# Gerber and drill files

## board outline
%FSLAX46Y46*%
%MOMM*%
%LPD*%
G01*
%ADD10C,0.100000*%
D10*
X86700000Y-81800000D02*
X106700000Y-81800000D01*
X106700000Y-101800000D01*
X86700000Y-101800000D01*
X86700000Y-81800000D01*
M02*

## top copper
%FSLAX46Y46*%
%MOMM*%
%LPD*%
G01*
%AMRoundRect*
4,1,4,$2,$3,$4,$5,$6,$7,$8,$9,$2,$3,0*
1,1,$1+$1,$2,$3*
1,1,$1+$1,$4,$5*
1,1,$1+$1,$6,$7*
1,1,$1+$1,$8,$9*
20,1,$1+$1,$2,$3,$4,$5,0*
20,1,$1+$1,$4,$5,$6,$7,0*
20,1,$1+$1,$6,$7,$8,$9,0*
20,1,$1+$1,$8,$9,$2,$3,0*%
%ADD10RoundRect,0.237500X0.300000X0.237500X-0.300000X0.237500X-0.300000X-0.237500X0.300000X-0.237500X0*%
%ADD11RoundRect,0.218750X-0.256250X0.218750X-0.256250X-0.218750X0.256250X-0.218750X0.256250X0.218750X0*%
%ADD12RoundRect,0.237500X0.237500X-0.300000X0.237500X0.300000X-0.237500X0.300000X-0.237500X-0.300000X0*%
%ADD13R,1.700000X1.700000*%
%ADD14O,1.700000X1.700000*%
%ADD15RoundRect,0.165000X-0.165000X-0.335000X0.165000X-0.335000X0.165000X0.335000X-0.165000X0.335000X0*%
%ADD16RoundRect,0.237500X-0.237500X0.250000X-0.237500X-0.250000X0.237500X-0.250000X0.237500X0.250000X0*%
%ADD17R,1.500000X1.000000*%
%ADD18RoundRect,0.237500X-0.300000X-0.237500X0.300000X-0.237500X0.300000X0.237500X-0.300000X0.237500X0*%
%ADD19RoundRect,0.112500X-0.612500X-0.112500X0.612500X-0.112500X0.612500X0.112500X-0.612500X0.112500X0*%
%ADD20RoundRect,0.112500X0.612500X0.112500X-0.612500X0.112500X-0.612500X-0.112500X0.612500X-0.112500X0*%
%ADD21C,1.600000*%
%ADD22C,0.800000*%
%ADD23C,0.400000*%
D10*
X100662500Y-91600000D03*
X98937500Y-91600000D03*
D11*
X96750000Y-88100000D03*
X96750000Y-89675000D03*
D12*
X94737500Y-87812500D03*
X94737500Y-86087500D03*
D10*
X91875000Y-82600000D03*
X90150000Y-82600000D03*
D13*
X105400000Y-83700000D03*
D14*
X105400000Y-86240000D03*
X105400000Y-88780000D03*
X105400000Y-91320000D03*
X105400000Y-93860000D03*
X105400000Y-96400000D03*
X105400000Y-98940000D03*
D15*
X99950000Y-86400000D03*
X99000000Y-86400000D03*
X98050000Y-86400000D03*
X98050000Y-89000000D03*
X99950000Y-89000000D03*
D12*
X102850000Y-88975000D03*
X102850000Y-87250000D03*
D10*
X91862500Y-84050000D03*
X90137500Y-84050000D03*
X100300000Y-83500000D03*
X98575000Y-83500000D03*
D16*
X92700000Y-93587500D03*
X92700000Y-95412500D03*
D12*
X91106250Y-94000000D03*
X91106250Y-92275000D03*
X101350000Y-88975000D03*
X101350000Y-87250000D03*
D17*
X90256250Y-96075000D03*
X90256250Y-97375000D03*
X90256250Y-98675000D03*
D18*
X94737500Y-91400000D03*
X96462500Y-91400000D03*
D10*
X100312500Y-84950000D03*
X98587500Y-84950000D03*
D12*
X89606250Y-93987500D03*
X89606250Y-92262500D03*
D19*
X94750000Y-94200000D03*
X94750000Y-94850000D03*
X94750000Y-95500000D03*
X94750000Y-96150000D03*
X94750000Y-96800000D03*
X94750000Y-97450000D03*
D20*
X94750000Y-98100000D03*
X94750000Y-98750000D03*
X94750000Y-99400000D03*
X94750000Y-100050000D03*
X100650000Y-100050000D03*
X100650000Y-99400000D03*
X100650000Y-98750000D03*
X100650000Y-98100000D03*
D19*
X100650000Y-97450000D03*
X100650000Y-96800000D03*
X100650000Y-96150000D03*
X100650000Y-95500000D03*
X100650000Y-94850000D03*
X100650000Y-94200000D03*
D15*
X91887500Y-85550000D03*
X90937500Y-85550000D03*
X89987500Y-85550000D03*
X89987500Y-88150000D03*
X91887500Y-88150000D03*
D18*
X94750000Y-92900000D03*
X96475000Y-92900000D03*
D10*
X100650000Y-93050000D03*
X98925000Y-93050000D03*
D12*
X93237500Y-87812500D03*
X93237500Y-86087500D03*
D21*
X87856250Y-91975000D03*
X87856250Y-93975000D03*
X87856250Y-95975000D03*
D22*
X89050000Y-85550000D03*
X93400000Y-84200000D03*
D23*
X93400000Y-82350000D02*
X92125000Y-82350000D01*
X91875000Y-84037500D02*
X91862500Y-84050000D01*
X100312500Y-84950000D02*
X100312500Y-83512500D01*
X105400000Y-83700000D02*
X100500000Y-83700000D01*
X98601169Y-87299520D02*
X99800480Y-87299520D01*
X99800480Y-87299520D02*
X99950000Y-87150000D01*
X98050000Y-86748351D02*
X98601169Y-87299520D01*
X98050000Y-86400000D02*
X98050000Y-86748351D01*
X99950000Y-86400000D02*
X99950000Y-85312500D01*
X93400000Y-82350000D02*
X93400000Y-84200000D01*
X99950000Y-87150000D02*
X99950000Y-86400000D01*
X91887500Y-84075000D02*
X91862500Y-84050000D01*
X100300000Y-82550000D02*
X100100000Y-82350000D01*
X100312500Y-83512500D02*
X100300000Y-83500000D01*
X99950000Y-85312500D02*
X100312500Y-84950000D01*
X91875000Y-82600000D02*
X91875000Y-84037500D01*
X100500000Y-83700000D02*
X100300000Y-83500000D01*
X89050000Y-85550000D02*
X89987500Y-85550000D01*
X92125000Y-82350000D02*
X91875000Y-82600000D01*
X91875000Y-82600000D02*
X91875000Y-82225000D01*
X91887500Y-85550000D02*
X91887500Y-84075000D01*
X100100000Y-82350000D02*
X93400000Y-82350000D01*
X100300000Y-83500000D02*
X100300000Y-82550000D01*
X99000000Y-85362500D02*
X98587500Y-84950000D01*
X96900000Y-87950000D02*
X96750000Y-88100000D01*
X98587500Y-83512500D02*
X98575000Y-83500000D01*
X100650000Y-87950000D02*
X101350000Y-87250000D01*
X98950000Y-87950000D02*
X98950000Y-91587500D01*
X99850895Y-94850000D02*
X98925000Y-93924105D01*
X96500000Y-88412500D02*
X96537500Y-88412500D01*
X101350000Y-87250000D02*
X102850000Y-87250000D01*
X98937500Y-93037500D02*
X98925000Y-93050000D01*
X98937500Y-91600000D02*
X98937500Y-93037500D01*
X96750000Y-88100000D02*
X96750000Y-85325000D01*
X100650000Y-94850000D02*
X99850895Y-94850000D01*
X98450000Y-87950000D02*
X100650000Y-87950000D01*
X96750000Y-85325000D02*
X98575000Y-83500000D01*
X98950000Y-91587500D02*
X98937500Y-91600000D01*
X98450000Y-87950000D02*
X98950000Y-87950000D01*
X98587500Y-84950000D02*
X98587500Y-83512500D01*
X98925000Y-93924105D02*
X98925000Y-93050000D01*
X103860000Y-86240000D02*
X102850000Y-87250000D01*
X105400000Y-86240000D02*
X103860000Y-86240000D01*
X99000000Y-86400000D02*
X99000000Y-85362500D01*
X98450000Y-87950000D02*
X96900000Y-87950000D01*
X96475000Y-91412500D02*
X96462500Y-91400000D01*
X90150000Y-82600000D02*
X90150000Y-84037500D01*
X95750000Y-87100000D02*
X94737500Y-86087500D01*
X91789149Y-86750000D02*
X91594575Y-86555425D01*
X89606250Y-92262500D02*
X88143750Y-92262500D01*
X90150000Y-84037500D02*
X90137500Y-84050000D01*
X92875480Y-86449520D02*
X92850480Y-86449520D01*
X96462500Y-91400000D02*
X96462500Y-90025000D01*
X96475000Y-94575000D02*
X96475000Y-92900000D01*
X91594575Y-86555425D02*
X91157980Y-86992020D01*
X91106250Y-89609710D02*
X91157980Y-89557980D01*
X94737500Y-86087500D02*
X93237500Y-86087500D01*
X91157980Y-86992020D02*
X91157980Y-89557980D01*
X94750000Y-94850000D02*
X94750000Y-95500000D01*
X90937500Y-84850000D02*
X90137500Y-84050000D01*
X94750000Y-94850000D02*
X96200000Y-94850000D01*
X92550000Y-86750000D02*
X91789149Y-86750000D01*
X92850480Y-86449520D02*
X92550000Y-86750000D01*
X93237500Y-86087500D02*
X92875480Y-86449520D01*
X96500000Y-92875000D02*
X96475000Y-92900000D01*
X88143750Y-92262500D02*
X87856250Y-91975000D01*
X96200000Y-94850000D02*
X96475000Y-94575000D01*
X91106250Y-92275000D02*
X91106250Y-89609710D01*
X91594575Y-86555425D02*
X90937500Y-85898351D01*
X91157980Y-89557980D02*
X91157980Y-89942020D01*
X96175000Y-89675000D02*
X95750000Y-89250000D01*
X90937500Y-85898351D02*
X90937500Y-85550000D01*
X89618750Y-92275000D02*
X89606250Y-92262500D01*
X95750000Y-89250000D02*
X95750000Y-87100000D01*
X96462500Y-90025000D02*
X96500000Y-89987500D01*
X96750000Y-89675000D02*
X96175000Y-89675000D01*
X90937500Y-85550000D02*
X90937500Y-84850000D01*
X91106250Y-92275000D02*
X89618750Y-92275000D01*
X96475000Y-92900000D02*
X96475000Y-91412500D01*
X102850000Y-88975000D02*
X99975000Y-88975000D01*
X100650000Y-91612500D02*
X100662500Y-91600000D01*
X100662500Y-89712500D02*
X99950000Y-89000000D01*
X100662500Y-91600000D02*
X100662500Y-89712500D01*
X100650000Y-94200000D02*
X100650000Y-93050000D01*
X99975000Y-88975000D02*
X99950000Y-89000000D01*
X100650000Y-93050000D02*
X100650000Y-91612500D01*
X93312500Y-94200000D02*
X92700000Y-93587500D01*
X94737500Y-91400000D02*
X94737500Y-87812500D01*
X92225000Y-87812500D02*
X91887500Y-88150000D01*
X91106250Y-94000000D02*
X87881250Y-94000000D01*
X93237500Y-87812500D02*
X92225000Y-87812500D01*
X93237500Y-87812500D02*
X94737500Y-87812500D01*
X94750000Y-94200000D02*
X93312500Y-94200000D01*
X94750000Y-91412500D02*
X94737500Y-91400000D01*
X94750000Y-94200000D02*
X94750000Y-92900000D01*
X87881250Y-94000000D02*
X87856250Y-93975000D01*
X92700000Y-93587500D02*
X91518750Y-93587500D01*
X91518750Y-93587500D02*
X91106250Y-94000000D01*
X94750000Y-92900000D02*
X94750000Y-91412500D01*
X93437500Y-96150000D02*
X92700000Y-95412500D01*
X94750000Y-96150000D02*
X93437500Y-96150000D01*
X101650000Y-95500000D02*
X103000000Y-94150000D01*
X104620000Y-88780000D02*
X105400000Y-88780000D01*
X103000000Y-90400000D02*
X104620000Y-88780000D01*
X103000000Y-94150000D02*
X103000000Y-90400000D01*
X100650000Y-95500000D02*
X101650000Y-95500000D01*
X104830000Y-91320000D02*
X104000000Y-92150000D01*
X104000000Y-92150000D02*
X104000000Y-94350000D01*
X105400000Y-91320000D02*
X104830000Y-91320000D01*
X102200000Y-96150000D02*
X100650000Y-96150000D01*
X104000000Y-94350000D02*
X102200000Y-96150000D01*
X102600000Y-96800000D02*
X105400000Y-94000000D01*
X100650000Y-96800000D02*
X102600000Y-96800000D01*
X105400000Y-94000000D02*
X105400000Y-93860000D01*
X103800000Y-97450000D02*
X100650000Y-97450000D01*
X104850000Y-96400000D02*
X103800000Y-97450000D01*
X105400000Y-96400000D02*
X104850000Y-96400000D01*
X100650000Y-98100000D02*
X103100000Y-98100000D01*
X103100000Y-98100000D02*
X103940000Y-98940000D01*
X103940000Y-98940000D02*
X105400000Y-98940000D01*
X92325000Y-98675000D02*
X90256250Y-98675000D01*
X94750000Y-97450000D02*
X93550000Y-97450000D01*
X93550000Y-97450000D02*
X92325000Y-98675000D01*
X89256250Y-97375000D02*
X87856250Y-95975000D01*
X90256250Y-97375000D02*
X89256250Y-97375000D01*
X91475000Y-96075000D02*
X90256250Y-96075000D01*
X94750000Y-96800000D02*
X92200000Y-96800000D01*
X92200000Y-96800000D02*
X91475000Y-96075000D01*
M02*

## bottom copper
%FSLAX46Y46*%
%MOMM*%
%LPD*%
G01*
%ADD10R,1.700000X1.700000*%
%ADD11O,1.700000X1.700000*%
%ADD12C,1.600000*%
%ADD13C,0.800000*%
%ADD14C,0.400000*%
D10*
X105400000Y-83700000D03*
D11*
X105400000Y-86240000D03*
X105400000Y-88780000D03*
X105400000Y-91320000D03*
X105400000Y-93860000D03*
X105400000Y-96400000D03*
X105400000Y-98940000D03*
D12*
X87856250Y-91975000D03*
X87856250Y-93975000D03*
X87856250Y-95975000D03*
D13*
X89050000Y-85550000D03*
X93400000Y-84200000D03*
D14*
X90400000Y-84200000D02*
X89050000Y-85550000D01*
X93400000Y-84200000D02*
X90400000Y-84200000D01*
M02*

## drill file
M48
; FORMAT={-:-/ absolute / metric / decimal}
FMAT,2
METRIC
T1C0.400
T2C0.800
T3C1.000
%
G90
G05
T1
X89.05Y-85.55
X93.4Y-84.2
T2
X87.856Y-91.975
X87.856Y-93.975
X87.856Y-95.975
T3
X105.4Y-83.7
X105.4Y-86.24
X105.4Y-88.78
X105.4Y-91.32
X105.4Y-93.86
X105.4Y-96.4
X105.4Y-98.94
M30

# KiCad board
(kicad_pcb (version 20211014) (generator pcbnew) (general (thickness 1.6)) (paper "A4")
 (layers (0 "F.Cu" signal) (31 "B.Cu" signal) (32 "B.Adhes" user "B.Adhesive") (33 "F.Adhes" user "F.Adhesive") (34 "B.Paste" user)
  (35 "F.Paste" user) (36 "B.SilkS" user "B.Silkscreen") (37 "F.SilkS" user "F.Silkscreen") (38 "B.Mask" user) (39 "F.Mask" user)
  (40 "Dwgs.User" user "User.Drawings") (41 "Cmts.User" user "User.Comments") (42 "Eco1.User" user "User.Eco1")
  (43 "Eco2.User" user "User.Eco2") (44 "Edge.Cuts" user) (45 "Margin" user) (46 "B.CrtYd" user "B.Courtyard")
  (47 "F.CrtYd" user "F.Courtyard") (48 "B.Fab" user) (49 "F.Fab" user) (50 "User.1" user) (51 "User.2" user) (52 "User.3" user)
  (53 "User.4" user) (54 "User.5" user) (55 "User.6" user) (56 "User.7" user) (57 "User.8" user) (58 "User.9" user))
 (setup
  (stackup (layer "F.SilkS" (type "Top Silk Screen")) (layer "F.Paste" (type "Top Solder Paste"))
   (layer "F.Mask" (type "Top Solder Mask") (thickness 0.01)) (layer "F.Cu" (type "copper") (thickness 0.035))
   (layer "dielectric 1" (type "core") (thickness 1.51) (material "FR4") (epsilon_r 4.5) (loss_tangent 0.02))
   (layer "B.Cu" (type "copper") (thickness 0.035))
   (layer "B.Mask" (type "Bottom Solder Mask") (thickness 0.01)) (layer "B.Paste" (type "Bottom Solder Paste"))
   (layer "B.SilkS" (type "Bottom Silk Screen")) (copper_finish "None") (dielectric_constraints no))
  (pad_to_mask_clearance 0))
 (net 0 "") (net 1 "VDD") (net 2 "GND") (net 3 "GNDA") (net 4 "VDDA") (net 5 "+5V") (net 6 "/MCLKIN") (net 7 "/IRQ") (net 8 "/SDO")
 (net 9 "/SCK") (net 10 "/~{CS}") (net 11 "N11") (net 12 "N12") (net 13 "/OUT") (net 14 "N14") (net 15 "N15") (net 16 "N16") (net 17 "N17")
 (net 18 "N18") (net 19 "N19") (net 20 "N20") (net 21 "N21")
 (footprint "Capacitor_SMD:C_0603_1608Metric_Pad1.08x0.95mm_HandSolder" (layer "F.Cu") (at 99.8 91.6 180)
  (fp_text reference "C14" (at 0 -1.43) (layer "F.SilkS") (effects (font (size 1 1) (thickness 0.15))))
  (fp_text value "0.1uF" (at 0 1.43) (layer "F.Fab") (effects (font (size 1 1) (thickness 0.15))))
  (pad "1" smd roundrect locked (at -0.8625 0 180) (size 1.075 0.95) (layers "F.Cu" "F.Paste" "F.Mask") (roundrect_rratio 0.25)
   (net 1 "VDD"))
  (pad "2" smd roundrect locked (at 0.8625 0 180) (size 1.075 0.95) (layers "F.Cu" "F.Paste" "F.Mask") (roundrect_rratio 0.25) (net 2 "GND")))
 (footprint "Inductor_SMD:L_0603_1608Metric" (layer "F.Cu") (at 96.75 88.8875 -90)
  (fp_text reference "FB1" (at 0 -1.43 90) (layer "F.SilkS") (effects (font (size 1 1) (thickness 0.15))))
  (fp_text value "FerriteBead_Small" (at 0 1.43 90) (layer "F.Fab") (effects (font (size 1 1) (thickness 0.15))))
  (pad "1" smd roundrect locked (at -0.7875 0 270) (size 0.875 0.95) (layers "F.Cu" "F.Paste" "F.Mask") (roundrect_rratio 0.25)
   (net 2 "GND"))
  (pad "2" smd roundrect locked (at 0.7875 0 270) (size 0.875 0.95) (layers "F.Cu" "F.Paste" "F.Mask") (roundrect_rratio 0.25)
   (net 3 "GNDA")))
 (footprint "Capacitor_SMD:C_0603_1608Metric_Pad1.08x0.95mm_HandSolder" (layer "F.Cu") (at 94.7375 86.95 90)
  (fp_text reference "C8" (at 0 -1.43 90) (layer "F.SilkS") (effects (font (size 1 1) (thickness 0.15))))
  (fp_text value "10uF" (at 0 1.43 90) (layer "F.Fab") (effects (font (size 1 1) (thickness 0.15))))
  (pad "1" smd roundrect locked (at -0.8625 0 90) (size 1.075 0.95) (layers "F.Cu" "F.Paste" "F.Mask") (roundrect_rratio 0.25)
   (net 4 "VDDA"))
  (pad "2" smd roundrect locked (at 0.8625 0 90) (size 1.075 0.95) (layers "F.Cu" "F.Paste" "F.Mask") (roundrect_rratio 0.25) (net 3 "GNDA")))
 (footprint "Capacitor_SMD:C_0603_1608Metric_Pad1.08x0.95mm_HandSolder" (layer "F.Cu") (at 91.0125 82.6 180)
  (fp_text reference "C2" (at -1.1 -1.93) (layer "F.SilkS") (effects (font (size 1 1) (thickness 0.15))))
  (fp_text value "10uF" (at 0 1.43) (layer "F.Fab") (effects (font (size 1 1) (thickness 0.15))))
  (pad "1" smd roundrect locked (at -0.8625 0 180) (size 1.075 0.95) (layers "F.Cu" "F.Paste" "F.Mask") (roundrect_rratio 0.25)
   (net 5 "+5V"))
  (pad "2" smd roundrect locked (at 0.8625 0 180) (size 1.075 0.95) (layers "F.Cu" "F.Paste" "F.Mask") (roundrect_rratio 0.25)
   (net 3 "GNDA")))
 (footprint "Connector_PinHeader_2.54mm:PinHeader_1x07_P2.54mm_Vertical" (layer "F.Cu") (at 105.4 83.7)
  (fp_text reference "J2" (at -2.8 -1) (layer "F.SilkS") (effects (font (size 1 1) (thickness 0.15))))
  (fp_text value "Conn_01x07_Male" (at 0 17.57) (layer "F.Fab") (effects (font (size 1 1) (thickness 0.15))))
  (pad "1" thru_hole rect locked (at 0 0) (size 1.7 1.7) (drill 1) (layers *.Cu *.Mask) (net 5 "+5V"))
  (pad "2" thru_hole oval locked (at 0 2.54) (size 1.7 1.7) (drill 1) (layers *.Cu *.Mask) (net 2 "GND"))
  (pad "3" thru_hole oval locked (at 0 5.08) (size 1.7 1.7) (drill 1) (layers *.Cu *.Mask) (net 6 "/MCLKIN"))
  (pad "4" thru_hole oval locked (at 0 7.62) (size 1.7 1.7) (drill 1) (layers *.Cu *.Mask) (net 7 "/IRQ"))
  (pad "5" thru_hole oval locked (at 0 10.16) (size 1.7 1.7) (drill 1) (layers *.Cu *.Mask) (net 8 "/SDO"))
  (pad "6" thru_hole oval locked (at 0 12.7) (size 1.7 1.7) (drill 1) (layers *.Cu *.Mask) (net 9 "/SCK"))
  (pad "7" thru_hole oval locked (at 0 15.24) (size 1.7 1.7) (drill 1) (layers *.Cu *.Mask) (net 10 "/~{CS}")))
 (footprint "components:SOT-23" (layer "F.Cu") (at 99 89)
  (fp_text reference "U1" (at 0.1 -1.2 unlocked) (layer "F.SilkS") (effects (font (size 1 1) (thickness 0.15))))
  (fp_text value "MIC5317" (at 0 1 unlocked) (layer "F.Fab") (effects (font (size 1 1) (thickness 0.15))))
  (pad "1" smd roundrect (at 0.95 -2.6) (size 0.66 1) (layers "F.Cu" "F.Paste" "F.Mask") (roundrect_rratio 0.25) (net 5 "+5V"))
  (pad "2" smd roundrect (at 0 -2.6) (size 0.66 1) (layers "F.Cu" "F.Paste" "F.Mask") (roundrect_rratio 0.25) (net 2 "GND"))
  (pad "3" smd roundrect (at -0.95 -2.6) (size 0.66 1) (layers "F.Cu" "F.Paste" "F.Mask") (roundrect_rratio 0.25) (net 5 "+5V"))
  (pad "4" smd roundrect (at -0.95 0) (size 0.66 1) (layers "F.Cu" "F.Paste" "F.Mask") (roundrect_rratio 0.25))
  (pad "5" smd roundrect (at 0.95 0) (size 0.66 1) (layers "F.Cu" "F.Paste" "F.Mask") (roundrect_rratio 0.25) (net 1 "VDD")))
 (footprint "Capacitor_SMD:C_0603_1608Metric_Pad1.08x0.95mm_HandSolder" (layer "F.Cu") (at 102.85 88.1125 90)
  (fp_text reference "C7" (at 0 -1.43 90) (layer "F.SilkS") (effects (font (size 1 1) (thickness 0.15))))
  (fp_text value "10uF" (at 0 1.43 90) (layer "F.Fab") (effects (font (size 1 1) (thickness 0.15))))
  (pad "1" smd roundrect locked (at -0.8625 0 90) (size 1.075 0.95) (layers "F.Cu" "F.Paste" "F.Mask") (roundrect_rratio 0.25) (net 1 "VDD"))
  (pad "2" smd roundrect locked (at 0.8625 0 90) (size 1.075 0.95) (layers "F.Cu" "F.Paste" "F.Mask") (roundrect_rratio 0.25) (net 2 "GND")))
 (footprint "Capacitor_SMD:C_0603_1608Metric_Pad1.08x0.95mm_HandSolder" (layer "F.Cu") (at 91 84.05 180)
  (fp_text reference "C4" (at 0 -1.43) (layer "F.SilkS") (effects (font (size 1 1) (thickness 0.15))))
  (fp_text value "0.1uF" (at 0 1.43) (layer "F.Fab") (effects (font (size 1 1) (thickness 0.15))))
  (pad "1" smd roundrect locked (at -0.8625 0 180) (size 1.075 0.95) (layers "F.Cu" "F.Paste" "F.Mask") (roundrect_rratio 0.25)
   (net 5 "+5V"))
  (pad "2" smd roundrect locked (at 0.8625 0 180) (size 1.075 0.95) (layers "F.Cu" "F.Paste" "F.Mask") (roundrect_rratio 0.25)
   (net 3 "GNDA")))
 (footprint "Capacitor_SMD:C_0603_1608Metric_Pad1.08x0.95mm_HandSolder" (layer "F.Cu") (at 99.4375 83.5 180)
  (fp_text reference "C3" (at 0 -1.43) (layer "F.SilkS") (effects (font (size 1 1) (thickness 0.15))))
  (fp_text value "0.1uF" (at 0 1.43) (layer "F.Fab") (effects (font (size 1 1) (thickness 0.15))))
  (pad "1" smd roundrect locked (at -0.8625 0 180) (size 1.075 0.95) (layers "F.Cu" "F.Paste" "F.Mask") (roundrect_rratio 0.25)
   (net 5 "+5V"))
  (pad "2" smd roundrect locked (at 0.8625 0 180) (size 1.075 0.95) (layers "F.Cu" "F.Paste" "F.Mask") (roundrect_rratio 0.25) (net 2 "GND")))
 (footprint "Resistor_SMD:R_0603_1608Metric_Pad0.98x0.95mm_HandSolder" (layer "F.Cu") (at 92.7 94.5 -90)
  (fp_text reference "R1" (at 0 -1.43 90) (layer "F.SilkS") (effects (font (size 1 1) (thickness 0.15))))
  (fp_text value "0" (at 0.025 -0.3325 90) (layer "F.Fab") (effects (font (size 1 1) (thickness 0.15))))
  (pad "1" smd roundrect locked (at -0.9125 0 270) (size 0.975 0.95) (layers "F.Cu" "F.Paste" "F.Mask") (roundrect_rratio 0.25)
   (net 4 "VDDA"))
  (pad "2" smd roundrect locked (at 0.9125 0 270) (size 0.975 0.95) (layers "F.Cu" "F.Paste" "F.Mask") (roundrect_rratio 0.25)
   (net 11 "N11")))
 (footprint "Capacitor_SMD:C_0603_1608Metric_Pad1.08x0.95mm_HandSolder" (layer "F.Cu") (at 91.10625 93.1375 90)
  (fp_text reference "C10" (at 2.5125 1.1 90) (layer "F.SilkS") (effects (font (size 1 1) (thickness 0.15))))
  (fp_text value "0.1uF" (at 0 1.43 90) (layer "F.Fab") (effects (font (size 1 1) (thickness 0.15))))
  (pad "1" smd roundrect locked (at -0.8625 0 90) (size 1.075 0.95) (layers "F.Cu" "F.Paste" "F.Mask") (roundrect_rratio 0.25)
   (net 4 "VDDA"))
  (pad "2" smd roundrect locked (at 0.8625 0 90) (size 1.075 0.95) (layers "F.Cu" "F.Paste" "F.Mask") (roundrect_rratio 0.25) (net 3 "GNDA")))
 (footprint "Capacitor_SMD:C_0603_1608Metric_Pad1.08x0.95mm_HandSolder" (layer "F.Cu") (at 101.35 88.1125 90)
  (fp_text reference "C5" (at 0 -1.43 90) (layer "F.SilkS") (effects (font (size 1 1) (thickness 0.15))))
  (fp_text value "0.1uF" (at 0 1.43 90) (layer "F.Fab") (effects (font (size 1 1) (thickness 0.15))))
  (pad "1" smd roundrect locked (at -0.8625 0 90) (size 1.075 0.95) (layers "F.Cu" "F.Paste" "F.Mask") (roundrect_rratio 0.25) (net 1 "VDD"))
  (pad "2" smd roundrect locked (at 0.8625 0 90) (size 1.075 0.95) (layers "F.Cu" "F.Paste" "F.Mask") (roundrect_rratio 0.25) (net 2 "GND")))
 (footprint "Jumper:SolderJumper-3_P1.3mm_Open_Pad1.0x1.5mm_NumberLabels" (layer "F.Cu") (at 90.25625 97.375 -90)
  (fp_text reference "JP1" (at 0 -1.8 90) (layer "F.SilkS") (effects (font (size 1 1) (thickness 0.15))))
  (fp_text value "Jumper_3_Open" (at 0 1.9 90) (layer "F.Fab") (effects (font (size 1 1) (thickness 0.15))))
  (pad "1" smd rect locked (at -1.3 0 270) (size 1 1.5) (layers "F.Cu" "F.Mask") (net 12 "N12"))
  (pad "2" smd rect locked (at 0 0 270) (size 1 1.5) (layers "F.Cu" "F.Mask") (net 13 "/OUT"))
  (pad "3" smd rect locked (at 1.3 0 270) (size 1 1.5) (layers "F.Cu" "F.Mask") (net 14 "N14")))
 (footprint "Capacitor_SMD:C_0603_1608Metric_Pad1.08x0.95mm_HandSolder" (layer "F.Cu") (at 95.6 91.4)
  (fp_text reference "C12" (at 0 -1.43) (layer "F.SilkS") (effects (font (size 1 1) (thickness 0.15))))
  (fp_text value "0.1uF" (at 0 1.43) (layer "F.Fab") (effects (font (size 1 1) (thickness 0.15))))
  (pad "1" smd roundrect locked (at -0.8625 0) (size 1.075 0.95) (layers "F.Cu" "F.Paste" "F.Mask") (roundrect_rratio 0.25) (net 4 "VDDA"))
  (pad "2" smd roundrect locked (at 0.8625 0) (size 1.075 0.95) (layers "F.Cu" "F.Paste" "F.Mask") (roundrect_rratio 0.25) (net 3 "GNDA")))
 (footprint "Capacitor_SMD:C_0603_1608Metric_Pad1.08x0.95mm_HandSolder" (layer "F.Cu") (at 99.45 84.95 180)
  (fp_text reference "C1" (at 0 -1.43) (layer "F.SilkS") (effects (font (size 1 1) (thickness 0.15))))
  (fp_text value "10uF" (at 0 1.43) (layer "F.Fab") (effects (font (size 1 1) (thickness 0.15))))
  (pad "1" smd roundrect locked (at -0.8625 0 180) (size 1.075 0.95) (layers "F.Cu" "F.Paste" "F.Mask") (roundrect_rratio 0.25)
   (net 5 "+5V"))
  (pad "2" smd roundrect locked (at 0.8625 0 180) (size 1.075 0.95) (layers "F.Cu" "F.Paste" "F.Mask") (roundrect_rratio 0.25) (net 2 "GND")))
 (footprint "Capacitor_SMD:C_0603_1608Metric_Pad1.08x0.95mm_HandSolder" (layer "F.Cu") (at 89.60625 93.125 90)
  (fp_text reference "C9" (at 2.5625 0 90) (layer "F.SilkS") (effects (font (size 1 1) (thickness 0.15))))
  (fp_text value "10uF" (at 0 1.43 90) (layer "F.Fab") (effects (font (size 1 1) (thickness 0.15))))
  (pad "1" smd roundrect locked (at -0.8625 0 90) (size 1.075 0.95) (layers "F.Cu" "F.Paste" "F.Mask") (roundrect_rratio 0.25)
   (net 4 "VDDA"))
  (pad "2" smd roundrect locked (at 0.8625 0 90) (size 1.075 0.95) (layers "F.Cu" "F.Paste" "F.Mask") (roundrect_rratio 0.25) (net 3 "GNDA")))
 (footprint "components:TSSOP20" (layer "F.Cu") (at 97.7 97)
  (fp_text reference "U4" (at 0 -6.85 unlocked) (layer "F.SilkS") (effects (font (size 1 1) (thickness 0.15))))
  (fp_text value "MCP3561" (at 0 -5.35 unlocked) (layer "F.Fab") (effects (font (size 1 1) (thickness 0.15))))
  (pad "1" smd roundrect (at -2.95 -2.8) (size 1.45 0.45) (layers "F.Cu" "F.Paste" "F.Mask") (roundrect_rratio 0.25) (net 4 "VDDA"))
  (pad "2" smd roundrect (at -2.95 -2.15) (size 1.45 0.45) (layers "F.Cu" "F.Paste" "F.Mask") (roundrect_rratio 0.25) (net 3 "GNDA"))
  (pad "3" smd roundrect (at -2.95 -1.5) (size 1.45 0.45) (layers "F.Cu" "F.Paste" "F.Mask") (roundrect_rratio 0.25) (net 3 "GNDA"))
  (pad "4" smd roundrect (at -2.95 -0.85) (size 1.45 0.45) (layers "F.Cu" "F.Paste" "F.Mask") (roundrect_rratio 0.25) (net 11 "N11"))
  (pad "5" smd roundrect (at -2.95 -0.2) (size 1.45 0.45) (layers "F.Cu" "F.Paste" "F.Mask") (roundrect_rratio 0.25) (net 12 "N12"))
  (pad "6" smd roundrect (at -2.95 0.45) (size 1.45 0.45) (layers "F.Cu" "F.Paste" "F.Mask") (roundrect_rratio 0.25) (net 14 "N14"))
  (pad "7" smd roundrect (at -2.95 1.1 180) (size 1.45 0.45) (layers "F.Cu" "F.Paste" "F.Mask") (roundrect_rratio 0.25) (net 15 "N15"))
  (pad "8" smd roundrect (at -2.95 1.75 180) (size 1.45 0.45) (layers "F.Cu" "F.Paste" "F.Mask") (roundrect_rratio 0.25) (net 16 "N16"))
  (pad "9" smd roundrect (at -2.95 2.4 180) (size 1.45 0.45) (layers "F.Cu" "F.Paste" "F.Mask") (roundrect_rratio 0.25) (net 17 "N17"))
  (pad "10" smd roundrect (at -2.95 3.05 180) (size 1.45 0.45) (layers "F.Cu" "F.Paste" "F.Mask") (roundrect_rratio 0.25) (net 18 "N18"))
  (pad "11" smd roundrect (at 2.95 3.05 180) (size 1.45 0.45) (layers "F.Cu" "F.Paste" "F.Mask") (roundrect_rratio 0.25) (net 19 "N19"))
  (pad "12" smd roundrect (at 2.95 2.4 180) (size 1.45 0.45) (layers "F.Cu" "F.Paste" "F.Mask") (roundrect_rratio 0.25) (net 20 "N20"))
  (pad "13" smd roundrect (at 2.95 1.75 180) (size 1.45 0.45) (layers "F.Cu" "F.Paste" "F.Mask") (roundrect_rratio 0.25) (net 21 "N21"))
  (pad "14" smd roundrect (at 2.95 1.1 180) (size 1.45 0.45) (layers "F.Cu" "F.Paste" "F.Mask") (roundrect_rratio 0.25) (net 10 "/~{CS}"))
  (pad "15" smd roundrect (at 2.95 0.45) (size 1.45 0.45) (layers "F.Cu" "F.Paste" "F.Mask") (roundrect_rratio 0.25) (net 9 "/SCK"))
  (pad "16" smd roundrect (at 2.95 -0.2) (size 1.45 0.45) (layers "F.Cu" "F.Paste" "F.Mask") (roundrect_rratio 0.25) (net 8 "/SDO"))
  (pad "17" smd roundrect (at 2.95 -0.85) (size 1.45 0.45) (layers "F.Cu" "F.Paste" "F.Mask") (roundrect_rratio 0.25) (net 7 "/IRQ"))
  (pad "18" smd roundrect (at 2.95 -1.5) (size 1.45 0.45) (layers "F.Cu" "F.Paste" "F.Mask") (roundrect_rratio 0.25) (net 6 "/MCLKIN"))
  (pad "19" smd roundrect (at 2.95 -2.15) (size 1.45 0.45) (layers "F.Cu" "F.Paste" "F.Mask") (roundrect_rratio 0.25) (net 2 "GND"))
  (pad "20" smd roundrect (at 2.95 -2.8) (size 1.45 0.45) (layers "F.Cu" "F.Paste" "F.Mask") (roundrect_rratio 0.25) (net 1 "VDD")))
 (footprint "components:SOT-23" (layer "F.Cu") (at 90.9375 88.15)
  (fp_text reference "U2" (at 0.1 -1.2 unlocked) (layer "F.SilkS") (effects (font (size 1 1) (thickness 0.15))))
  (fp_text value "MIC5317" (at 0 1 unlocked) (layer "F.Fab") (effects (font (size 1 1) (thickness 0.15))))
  (pad "1" smd roundrect (at 0.95 -2.6) (size 0.66 1) (layers "F.Cu" "F.Paste" "F.Mask") (roundrect_rratio 0.25) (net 5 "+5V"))
  (pad "2" smd roundrect (at 0 -2.6) (size 0.66 1) (layers "F.Cu" "F.Paste" "F.Mask") (roundrect_rratio 0.25) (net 3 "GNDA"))
  (pad "3" smd roundrect (at -0.95 -2.6) (size 0.66 1) (layers "F.Cu" "F.Paste" "F.Mask") (roundrect_rratio 0.25) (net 5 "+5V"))
  (pad "4" smd roundrect (at -0.95 0) (size 0.66 1) (layers "F.Cu" "F.Paste" "F.Mask") (roundrect_rratio 0.25))
  (pad "5" smd roundrect (at 0.95 0) (size 0.66 1) (layers "F.Cu" "F.Paste" "F.Mask") (roundrect_rratio 0.25) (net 4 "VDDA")))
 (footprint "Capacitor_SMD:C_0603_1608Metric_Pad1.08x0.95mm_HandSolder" (layer "F.Cu") (at 95.6125 92.9)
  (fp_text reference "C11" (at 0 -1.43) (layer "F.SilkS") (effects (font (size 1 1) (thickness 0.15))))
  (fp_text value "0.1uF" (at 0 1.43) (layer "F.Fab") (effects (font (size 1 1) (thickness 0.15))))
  (pad "1" smd roundrect locked (at -0.8625 0) (size 1.075 0.95) (layers "F.Cu" "F.Paste" "F.Mask") (roundrect_rratio 0.25) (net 4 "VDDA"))
  (pad "2" smd roundrect locked (at 0.8625 0) (size 1.075 0.95) (layers "F.Cu" "F.Paste" "F.Mask") (roundrect_rratio 0.25) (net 3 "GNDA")))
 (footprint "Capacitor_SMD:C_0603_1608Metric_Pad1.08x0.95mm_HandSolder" (layer "F.Cu") (at 99.7875 93.05 180)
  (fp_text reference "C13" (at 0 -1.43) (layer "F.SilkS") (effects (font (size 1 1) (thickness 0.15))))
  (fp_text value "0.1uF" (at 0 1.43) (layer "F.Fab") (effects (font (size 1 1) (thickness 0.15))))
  (pad "1" smd roundrect locked (at -0.8625 0 180) (size 1.075 0.95) (layers "F.Cu" "F.Paste" "F.Mask") (roundrect_rratio 0.25)
   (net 1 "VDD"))
  (pad "2" smd roundrect locked (at 0.8625 0 180) (size 1.075 0.95) (layers "F.Cu" "F.Paste" "F.Mask") (roundrect_rratio 0.25) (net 2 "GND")))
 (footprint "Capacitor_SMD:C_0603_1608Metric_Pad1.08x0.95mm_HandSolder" (layer "F.Cu") (at 93.2375 86.95 90)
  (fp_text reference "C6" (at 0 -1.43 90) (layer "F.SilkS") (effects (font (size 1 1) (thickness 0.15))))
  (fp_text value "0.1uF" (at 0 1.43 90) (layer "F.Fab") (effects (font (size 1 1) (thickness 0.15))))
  (pad "1" smd roundrect locked (at -0.8625 0 90) (size 1.075 0.95) (layers "F.Cu" "F.Paste" "F.Mask") (roundrect_rratio 0.25)
   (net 4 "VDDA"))
  (pad "2" smd roundrect locked (at 0.8625 0 90) (size 1.075 0.95) (layers "F.Cu" "F.Paste" "F.Mask") (roundrect_rratio 0.25) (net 3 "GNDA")))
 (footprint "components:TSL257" (layer "B.Cu") (at 87.85625 93.975 -90)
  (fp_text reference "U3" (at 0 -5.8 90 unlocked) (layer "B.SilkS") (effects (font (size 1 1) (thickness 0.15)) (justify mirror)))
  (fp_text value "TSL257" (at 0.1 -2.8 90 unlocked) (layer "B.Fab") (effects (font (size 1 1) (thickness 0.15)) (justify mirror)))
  (pad "1" thru_hole circle (at -2 0 270) (size 1.6 1.6) (drill 0.8) (layers *.Cu *.Mask) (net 3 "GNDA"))
  (pad "2" thru_hole circle (at 0 0 270) (size 1.6 1.6) (drill 0.8) (layers *.Cu *.Mask) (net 4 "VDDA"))
  (pad "3" thru_hole circle (at 2 0 270) (size 1.6 1.6) (drill 0.8) (layers *.Cu *.Mask) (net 13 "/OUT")))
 (gr_rect (start 106.7 101.8) (end 86.7 81.8) (layer "Edge.Cuts") (width 0.1) (fill none))
 (segment (start 93.4 82.35) (end 92.125 82.35) (width 0.4) (layer "F.Cu") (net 5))
 (segment (start 91.875 84.0375) (end 91.8625 84.05) (width 0.4) (layer "F.Cu") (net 5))
 (segment (start 100.3125 84.95) (end 100.3125 83.5125) (width 0.4) (layer "F.Cu") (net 5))
 (segment (start 105.4 83.7) (end 100.5 83.7) (width 0.4) (layer "F.Cu") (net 5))
 (segment (start 98.601169 87.29952) (end 99.80048 87.29952) (width 0.4) (layer "F.Cu") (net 5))
 (segment (start 99.80048 87.29952) (end 99.95 87.15) (width 0.4) (layer "F.Cu") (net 5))
 (segment (start 98.05 86.748351) (end 98.601169 87.29952) (width 0.4) (layer "F.Cu") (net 5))
 (segment (start 98.05 86.4) (end 98.05 86.748351) (width 0.4) (layer "F.Cu") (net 5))
 (segment (start 99.95 86.4) (end 99.95 85.3125) (width 0.4) (layer "F.Cu") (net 5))
 (segment (start 93.4 82.35) (end 93.4 84.2) (width 0.4) (layer "F.Cu") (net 5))
 (segment (start 99.95 87.15) (end 99.95 86.4) (width 0.4) (layer "F.Cu") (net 5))
 (segment (start 91.8875 84.075) (end 91.8625 84.05) (width 0.4) (layer "F.Cu") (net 5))
 (segment (start 100.3 82.55) (end 100.1 82.35) (width 0.4) (layer "F.Cu") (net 5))
 (segment (start 100.3125 83.5125) (end 100.3 83.5) (width 0.4) (layer "F.Cu") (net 5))
 (segment (start 99.95 85.3125) (end 100.3125 84.95) (width 0.4) (layer "F.Cu") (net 5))
 (segment (start 91.875 82.6) (end 91.875 84.0375) (width 0.4) (layer "F.Cu") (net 5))
 (segment (start 100.5 83.7) (end 100.3 83.5) (width 0.4) (layer "F.Cu") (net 5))
 (segment (start 89.05 85.55) (end 89.9875 85.55) (width 0.4) (layer "F.Cu") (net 5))
 (segment (start 92.125 82.35) (end 91.875 82.6) (width 0.4) (layer "F.Cu") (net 5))
 (segment (start 91.875 82.6) (end 91.875 82.225) (width 0.4) (layer "F.Cu") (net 5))
 (segment (start 91.8875 85.55) (end 91.8875 84.075) (width 0.4) (layer "F.Cu") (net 5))
 (segment (start 100.1 82.35) (end 93.4 82.35) (width 0.4) (layer "F.Cu") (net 5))
 (segment (start 100.3 83.5) (end 100.3 82.55) (width 0.4) (layer "F.Cu") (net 5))
 (via (at 89.05 85.55) (size 0.8) (drill 0.4) (layers "F.Cu" "B.Cu") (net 5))
 (via (at 93.4 84.2) (size 0.8) (drill 0.4) (layers "F.Cu" "B.Cu") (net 5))
 (segment (start 90.4 84.2) (end 89.05 85.55) (width 0.4) (layer "B.Cu") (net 5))
 (segment (start 93.4 84.2) (end 90.4 84.2) (width 0.4) (layer "B.Cu") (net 5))
 (segment (start 99 85.3625) (end 98.5875 84.95) (width 0.4) (layer "F.Cu") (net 2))
 (segment (start 96.9 87.95) (end 96.75 88.1) (width 0.4) (layer "F.Cu") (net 2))
 (segment (start 98.5875 83.5125) (end 98.575 83.5) (width 0.4) (layer "F.Cu") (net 2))
 (segment (start 100.65 87.95) (end 101.35 87.25) (width 0.4) (layer "F.Cu") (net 2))
 (segment (start 98.95 87.95) (end 98.95 91.5875) (width 0.4) (layer "F.Cu") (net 2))
 (segment (start 99.850895 94.85) (end 98.925 93.924105) (width 0.4) (layer "F.Cu") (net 2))
 (segment (start 96.5 88.4125) (end 96.5375 88.4125) (width 0.4) (layer "F.Cu") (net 2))
 (segment (start 101.35 87.25) (end 102.85 87.25) (width 0.4) (layer "F.Cu") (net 2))
 (segment (start 98.9375 93.0375) (end 98.925 93.05) (width 0.4) (layer "F.Cu") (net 2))
 (segment (start 98.9375 91.6) (end 98.9375 93.0375) (width 0.4) (layer "F.Cu") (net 2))
 (segment (start 96.75 88.1) (end 96.75 85.325) (width 0.4) (layer "F.Cu") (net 2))
 (segment (start 100.65 94.85) (end 99.850895 94.85) (width 0.4) (layer "F.Cu") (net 2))
 (segment (start 98.45 87.95) (end 100.65 87.95) (width 0.4) (layer "F.Cu") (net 2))
 (segment (start 96.75 85.325) (end 98.575 83.5) (width 0.4) (layer "F.Cu") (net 2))
 (segment (start 98.95 91.5875) (end 98.9375 91.6) (width 0.4) (layer "F.Cu") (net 2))
 (segment (start 98.45 87.95) (end 98.95 87.95) (width 0.4) (layer "F.Cu") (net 2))
 (segment (start 98.5875 84.95) (end 98.5875 83.5125) (width 0.4) (layer "F.Cu") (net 2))
 (segment (start 98.925 93.924105) (end 98.925 93.05) (width 0.4) (layer "F.Cu") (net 2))
 (segment (start 103.86 86.24) (end 102.85 87.25) (width 0.4) (layer "F.Cu") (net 2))
 (segment (start 105.4 86.24) (end 103.86 86.24) (width 0.4) (layer "F.Cu") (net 2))
 (segment (start 99 86.4) (end 99 85.3625) (width 0.4) (layer "F.Cu") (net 2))
 (segment (start 98.45 87.95) (end 96.9 87.95) (width 0.4) (layer "F.Cu") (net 2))
 (segment (start 96.475 91.4125) (end 96.4625 91.4) (width 0.4) (layer "F.Cu") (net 3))
 (segment (start 90.15 82.6) (end 90.15 84.0375) (width 0.4) (layer "F.Cu") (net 3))
 (segment (start 95.75 87.1) (end 94.7375 86.0875) (width 0.4) (layer "F.Cu") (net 3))
 (segment (start 91.789149 86.75) (end 91.594575 86.555425) (width 0.4) (layer "F.Cu") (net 3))
 (segment (start 89.60625 92.2625) (end 88.14375 92.2625) (width 0.4) (layer "F.Cu") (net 3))
 (segment (start 90.15 84.0375) (end 90.1375 84.05) (width 0.4) (layer "F.Cu") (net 3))
 (segment (start 92.87548 86.44952) (end 92.85048 86.44952) (width 0.4) (layer "F.Cu") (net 3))
 (segment (start 96.4625 91.4) (end 96.4625 90.025) (width 0.4) (layer "F.Cu") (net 3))
 (segment (start 96.475 94.575) (end 96.475 92.9) (width 0.4) (layer "F.Cu") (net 3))
 (segment (start 91.594575 86.555425) (end 91.15798 86.99202) (width 0.4) (layer "F.Cu") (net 3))
 (segment (start 91.10625 89.60971) (end 91.15798 89.55798) (width 0.4) (layer "F.Cu") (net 3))
 (segment (start 94.7375 86.0875) (end 93.2375 86.0875) (width 0.4) (layer "F.Cu") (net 3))
 (segment (start 91.15798 86.99202) (end 91.15798 89.55798) (width 0.4) (layer "F.Cu") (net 3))
 (segment (start 94.75 94.85) (end 94.75 95.5) (width 0.4) (layer "F.Cu") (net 3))
 (segment (start 90.9375 84.85) (end 90.1375 84.05) (width 0.4) (layer "F.Cu") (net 3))
 (segment (start 94.75 94.85) (end 96.2 94.85) (width 0.4) (layer "F.Cu") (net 3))
 (segment (start 92.55 86.75) (end 91.789149 86.75) (width 0.4) (layer "F.Cu") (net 3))
 (segment (start 92.85048 86.44952) (end 92.55 86.75) (width 0.4) (layer "F.Cu") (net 3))
 (segment (start 93.2375 86.0875) (end 92.87548 86.44952) (width 0.4) (layer "F.Cu") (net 3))
 (segment (start 96.5 92.875) (end 96.475 92.9) (width 0.4) (layer "F.Cu") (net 3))
 (segment (start 88.14375 92.2625) (end 87.85625 91.975) (width 0.4) (layer "F.Cu") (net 3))
 (segment (start 96.2 94.85) (end 96.475 94.575) (width 0.4) (layer "F.Cu") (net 3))
 (segment (start 91.10625 92.275) (end 91.10625 89.60971) (width 0.4) (layer "F.Cu") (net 3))
 (segment (start 91.594575 86.555425) (end 90.9375 85.898351) (width 0.4) (layer "F.Cu") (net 3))
 (segment (start 91.15798 89.55798) (end 91.15798 89.94202) (width 0.4) (layer "F.Cu") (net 3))
 (segment (start 96.175 89.675) (end 95.75 89.25) (width 0.4) (layer "F.Cu") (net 3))
 (segment (start 90.9375 85.898351) (end 90.9375 85.55) (width 0.4) (layer "F.Cu") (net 3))
 (segment (start 89.61875 92.275) (end 89.60625 92.2625) (width 0.4) (layer "F.Cu") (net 3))
 (segment (start 95.75 89.25) (end 95.75 87.1) (width 0.4) (layer "F.Cu") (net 3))
 (segment (start 96.4625 90.025) (end 96.5 89.9875) (width 0.4) (layer "F.Cu") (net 3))
 (segment (start 96.75 89.675) (end 96.175 89.675) (width 0.4) (layer "F.Cu") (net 3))
 (segment (start 90.9375 85.55) (end 90.9375 84.85) (width 0.4) (layer "F.Cu") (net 3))
 (segment (start 91.10625 92.275) (end 89.61875 92.275) (width 0.4) (layer "F.Cu") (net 3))
 (segment (start 96.475 92.9) (end 96.475 91.4125) (width 0.4) (layer "F.Cu") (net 3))
 (segment (start 102.85 88.975) (end 99.975 88.975) (width 0.4) (layer "F.Cu") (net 1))
 (segment (start 100.65 91.6125) (end 100.6625 91.6) (width 0.4) (layer "F.Cu") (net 1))
 (segment (start 100.6625 89.7125) (end 99.95 89) (width 0.4) (layer "F.Cu") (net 1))
 (segment (start 100.6625 91.6) (end 100.6625 89.7125) (width 0.4) (layer "F.Cu") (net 1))
 (segment (start 100.65 94.2) (end 100.65 93.05) (width 0.4) (layer "F.Cu") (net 1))
 (segment (start 99.975 88.975) (end 99.95 89) (width 0.4) (layer "F.Cu") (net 1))
 (segment (start 100.65 93.05) (end 100.65 91.6125) (width 0.4) (layer "F.Cu") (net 1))
 (segment (start 93.3125 94.2) (end 92.7 93.5875) (width 0.4) (layer "F.Cu") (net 4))
 (segment (start 94.7375 91.4) (end 94.7375 87.8125) (width 0.4) (layer "F.Cu") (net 4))
 (segment (start 92.225 87.8125) (end 91.8875 88.15) (width 0.4) (layer "F.Cu") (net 4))
 (segment (start 91.10625 94) (end 87.88125 94) (width 0.4) (layer "F.Cu") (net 4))
 (segment (start 93.2375 87.8125) (end 92.225 87.8125) (width 0.4) (layer "F.Cu") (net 4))
 (segment (start 93.2375 87.8125) (end 94.7375 87.8125) (width 0.4) (layer "F.Cu") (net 4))
 (segment (start 94.75 94.2) (end 93.3125 94.2) (width 0.4) (layer "F.Cu") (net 4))
 (segment (start 94.75 91.4125) (end 94.7375 91.4) (width 0.4) (layer "F.Cu") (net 4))
 (segment (start 94.75 94.2) (end 94.75 92.9) (width 0.4) (layer "F.Cu") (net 4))
 (segment (start 87.88125 94) (end 87.85625 93.975) (width 0.4) (layer "F.Cu") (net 4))
 (segment (start 92.7 93.5875) (end 91.51875 93.5875) (width 0.4) (layer "F.Cu") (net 4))
 (segment (start 91.51875 93.5875) (end 91.10625 94) (width 0.4) (layer "F.Cu") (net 4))
 (segment (start 94.75 92.9) (end 94.75 91.4125) (width 0.4) (layer "F.Cu") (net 4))
 (segment (start 93.4375 96.15) (end 92.7 95.4125) (width 0.4) (layer "F.Cu") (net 11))
 (segment (start 94.75 96.15) (end 93.4375 96.15) (width 0.4) (layer "F.Cu") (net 11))
 (segment (start 101.65 95.5) (end 103 94.15) (width 0.4) (layer "F.Cu") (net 6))
 (segment (start 104.62 88.78) (end 105.4 88.78) (width 0.4) (layer "F.Cu") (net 6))
 (segment (start 103 90.4) (end 104.62 88.78) (width 0.4) (layer "F.Cu") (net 6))
 (segment (start 103 94.15) (end 103 90.4) (width 0.4) (layer "F.Cu") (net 6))
 (segment (start 100.65 95.5) (end 101.65 95.5) (width 0.4) (layer "F.Cu") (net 6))
 (segment (start 104.83 91.32) (end 104 92.15) (width 0.4) (layer "F.Cu") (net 7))
 (segment (start 104 92.15) (end 104 94.35) (width 0.4) (layer "F.Cu") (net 7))
 (segment (start 105.4 91.32) (end 104.83 91.32) (width 0.4) (layer "F.Cu") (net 7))
 (segment (start 102.2 96.15) (end 100.65 96.15) (width 0.4) (layer "F.Cu") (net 7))
 (segment (start 104 94.35) (end 102.2 96.15) (width 0.4) (layer "F.Cu") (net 7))
 (segment (start 102.6 96.8) (end 105.4 94) (width 0.4) (layer "F.Cu") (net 8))
 (segment (start 100.65 96.8) (end 102.6 96.8) (width 0.4) (layer "F.Cu") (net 8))
 (segment (start 105.4 94) (end 105.4 93.86) (width 0.4) (layer "F.Cu") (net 8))
 (segment (start 103.8 97.45) (end 100.65 97.45) (width 0.4) (layer "F.Cu") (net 9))
 (segment (start 104.85 96.4) (end 103.8 97.45) (width 0.4) (layer "F.Cu") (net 9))
 (segment (start 105.4 96.4) (end 104.85 96.4) (width 0.4) (layer "F.Cu") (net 9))
 (segment (start 100.65 98.1) (end 103.1 98.1) (width 0.4) (layer "F.Cu") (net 10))
 (segment (start 103.1 98.1) (end 103.94 98.94) (width 0.4) (layer "F.Cu") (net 10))
 (segment (start 103.94 98.94) (end 105.4 98.94) (width 0.4) (layer "F.Cu") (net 10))
 (segment (start 92.325 98.675) (end 90.25625 98.675) (width 0.4) (layer "F.Cu") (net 14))
 (segment (start 94.75 97.45) (end 93.55 97.45) (width 0.4) (layer "F.Cu") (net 14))
 (segment (start 93.55 97.45) (end 92.325 98.675) (width 0.4) (layer "F.Cu") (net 14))
 (segment (start 89.25625 97.375) (end 87.85625 95.975) (width 0.4) (layer "F.Cu") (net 13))
 (segment (start 90.25625 97.375) (end 89.25625 97.375) (width 0.4) (layer "F.Cu") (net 13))
 (segment (start 91.475 96.075) (end 90.25625 96.075) (width 0.4) (layer "F.Cu") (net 12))
 (segment (start 94.75 96.8) (end 92.2 96.8) (width 0.4) (layer "F.Cu") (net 12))
 (segment (start 92.2 96.8) (end 91.475 96.075) (width 0.4) (layer "F.Cu") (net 12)))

